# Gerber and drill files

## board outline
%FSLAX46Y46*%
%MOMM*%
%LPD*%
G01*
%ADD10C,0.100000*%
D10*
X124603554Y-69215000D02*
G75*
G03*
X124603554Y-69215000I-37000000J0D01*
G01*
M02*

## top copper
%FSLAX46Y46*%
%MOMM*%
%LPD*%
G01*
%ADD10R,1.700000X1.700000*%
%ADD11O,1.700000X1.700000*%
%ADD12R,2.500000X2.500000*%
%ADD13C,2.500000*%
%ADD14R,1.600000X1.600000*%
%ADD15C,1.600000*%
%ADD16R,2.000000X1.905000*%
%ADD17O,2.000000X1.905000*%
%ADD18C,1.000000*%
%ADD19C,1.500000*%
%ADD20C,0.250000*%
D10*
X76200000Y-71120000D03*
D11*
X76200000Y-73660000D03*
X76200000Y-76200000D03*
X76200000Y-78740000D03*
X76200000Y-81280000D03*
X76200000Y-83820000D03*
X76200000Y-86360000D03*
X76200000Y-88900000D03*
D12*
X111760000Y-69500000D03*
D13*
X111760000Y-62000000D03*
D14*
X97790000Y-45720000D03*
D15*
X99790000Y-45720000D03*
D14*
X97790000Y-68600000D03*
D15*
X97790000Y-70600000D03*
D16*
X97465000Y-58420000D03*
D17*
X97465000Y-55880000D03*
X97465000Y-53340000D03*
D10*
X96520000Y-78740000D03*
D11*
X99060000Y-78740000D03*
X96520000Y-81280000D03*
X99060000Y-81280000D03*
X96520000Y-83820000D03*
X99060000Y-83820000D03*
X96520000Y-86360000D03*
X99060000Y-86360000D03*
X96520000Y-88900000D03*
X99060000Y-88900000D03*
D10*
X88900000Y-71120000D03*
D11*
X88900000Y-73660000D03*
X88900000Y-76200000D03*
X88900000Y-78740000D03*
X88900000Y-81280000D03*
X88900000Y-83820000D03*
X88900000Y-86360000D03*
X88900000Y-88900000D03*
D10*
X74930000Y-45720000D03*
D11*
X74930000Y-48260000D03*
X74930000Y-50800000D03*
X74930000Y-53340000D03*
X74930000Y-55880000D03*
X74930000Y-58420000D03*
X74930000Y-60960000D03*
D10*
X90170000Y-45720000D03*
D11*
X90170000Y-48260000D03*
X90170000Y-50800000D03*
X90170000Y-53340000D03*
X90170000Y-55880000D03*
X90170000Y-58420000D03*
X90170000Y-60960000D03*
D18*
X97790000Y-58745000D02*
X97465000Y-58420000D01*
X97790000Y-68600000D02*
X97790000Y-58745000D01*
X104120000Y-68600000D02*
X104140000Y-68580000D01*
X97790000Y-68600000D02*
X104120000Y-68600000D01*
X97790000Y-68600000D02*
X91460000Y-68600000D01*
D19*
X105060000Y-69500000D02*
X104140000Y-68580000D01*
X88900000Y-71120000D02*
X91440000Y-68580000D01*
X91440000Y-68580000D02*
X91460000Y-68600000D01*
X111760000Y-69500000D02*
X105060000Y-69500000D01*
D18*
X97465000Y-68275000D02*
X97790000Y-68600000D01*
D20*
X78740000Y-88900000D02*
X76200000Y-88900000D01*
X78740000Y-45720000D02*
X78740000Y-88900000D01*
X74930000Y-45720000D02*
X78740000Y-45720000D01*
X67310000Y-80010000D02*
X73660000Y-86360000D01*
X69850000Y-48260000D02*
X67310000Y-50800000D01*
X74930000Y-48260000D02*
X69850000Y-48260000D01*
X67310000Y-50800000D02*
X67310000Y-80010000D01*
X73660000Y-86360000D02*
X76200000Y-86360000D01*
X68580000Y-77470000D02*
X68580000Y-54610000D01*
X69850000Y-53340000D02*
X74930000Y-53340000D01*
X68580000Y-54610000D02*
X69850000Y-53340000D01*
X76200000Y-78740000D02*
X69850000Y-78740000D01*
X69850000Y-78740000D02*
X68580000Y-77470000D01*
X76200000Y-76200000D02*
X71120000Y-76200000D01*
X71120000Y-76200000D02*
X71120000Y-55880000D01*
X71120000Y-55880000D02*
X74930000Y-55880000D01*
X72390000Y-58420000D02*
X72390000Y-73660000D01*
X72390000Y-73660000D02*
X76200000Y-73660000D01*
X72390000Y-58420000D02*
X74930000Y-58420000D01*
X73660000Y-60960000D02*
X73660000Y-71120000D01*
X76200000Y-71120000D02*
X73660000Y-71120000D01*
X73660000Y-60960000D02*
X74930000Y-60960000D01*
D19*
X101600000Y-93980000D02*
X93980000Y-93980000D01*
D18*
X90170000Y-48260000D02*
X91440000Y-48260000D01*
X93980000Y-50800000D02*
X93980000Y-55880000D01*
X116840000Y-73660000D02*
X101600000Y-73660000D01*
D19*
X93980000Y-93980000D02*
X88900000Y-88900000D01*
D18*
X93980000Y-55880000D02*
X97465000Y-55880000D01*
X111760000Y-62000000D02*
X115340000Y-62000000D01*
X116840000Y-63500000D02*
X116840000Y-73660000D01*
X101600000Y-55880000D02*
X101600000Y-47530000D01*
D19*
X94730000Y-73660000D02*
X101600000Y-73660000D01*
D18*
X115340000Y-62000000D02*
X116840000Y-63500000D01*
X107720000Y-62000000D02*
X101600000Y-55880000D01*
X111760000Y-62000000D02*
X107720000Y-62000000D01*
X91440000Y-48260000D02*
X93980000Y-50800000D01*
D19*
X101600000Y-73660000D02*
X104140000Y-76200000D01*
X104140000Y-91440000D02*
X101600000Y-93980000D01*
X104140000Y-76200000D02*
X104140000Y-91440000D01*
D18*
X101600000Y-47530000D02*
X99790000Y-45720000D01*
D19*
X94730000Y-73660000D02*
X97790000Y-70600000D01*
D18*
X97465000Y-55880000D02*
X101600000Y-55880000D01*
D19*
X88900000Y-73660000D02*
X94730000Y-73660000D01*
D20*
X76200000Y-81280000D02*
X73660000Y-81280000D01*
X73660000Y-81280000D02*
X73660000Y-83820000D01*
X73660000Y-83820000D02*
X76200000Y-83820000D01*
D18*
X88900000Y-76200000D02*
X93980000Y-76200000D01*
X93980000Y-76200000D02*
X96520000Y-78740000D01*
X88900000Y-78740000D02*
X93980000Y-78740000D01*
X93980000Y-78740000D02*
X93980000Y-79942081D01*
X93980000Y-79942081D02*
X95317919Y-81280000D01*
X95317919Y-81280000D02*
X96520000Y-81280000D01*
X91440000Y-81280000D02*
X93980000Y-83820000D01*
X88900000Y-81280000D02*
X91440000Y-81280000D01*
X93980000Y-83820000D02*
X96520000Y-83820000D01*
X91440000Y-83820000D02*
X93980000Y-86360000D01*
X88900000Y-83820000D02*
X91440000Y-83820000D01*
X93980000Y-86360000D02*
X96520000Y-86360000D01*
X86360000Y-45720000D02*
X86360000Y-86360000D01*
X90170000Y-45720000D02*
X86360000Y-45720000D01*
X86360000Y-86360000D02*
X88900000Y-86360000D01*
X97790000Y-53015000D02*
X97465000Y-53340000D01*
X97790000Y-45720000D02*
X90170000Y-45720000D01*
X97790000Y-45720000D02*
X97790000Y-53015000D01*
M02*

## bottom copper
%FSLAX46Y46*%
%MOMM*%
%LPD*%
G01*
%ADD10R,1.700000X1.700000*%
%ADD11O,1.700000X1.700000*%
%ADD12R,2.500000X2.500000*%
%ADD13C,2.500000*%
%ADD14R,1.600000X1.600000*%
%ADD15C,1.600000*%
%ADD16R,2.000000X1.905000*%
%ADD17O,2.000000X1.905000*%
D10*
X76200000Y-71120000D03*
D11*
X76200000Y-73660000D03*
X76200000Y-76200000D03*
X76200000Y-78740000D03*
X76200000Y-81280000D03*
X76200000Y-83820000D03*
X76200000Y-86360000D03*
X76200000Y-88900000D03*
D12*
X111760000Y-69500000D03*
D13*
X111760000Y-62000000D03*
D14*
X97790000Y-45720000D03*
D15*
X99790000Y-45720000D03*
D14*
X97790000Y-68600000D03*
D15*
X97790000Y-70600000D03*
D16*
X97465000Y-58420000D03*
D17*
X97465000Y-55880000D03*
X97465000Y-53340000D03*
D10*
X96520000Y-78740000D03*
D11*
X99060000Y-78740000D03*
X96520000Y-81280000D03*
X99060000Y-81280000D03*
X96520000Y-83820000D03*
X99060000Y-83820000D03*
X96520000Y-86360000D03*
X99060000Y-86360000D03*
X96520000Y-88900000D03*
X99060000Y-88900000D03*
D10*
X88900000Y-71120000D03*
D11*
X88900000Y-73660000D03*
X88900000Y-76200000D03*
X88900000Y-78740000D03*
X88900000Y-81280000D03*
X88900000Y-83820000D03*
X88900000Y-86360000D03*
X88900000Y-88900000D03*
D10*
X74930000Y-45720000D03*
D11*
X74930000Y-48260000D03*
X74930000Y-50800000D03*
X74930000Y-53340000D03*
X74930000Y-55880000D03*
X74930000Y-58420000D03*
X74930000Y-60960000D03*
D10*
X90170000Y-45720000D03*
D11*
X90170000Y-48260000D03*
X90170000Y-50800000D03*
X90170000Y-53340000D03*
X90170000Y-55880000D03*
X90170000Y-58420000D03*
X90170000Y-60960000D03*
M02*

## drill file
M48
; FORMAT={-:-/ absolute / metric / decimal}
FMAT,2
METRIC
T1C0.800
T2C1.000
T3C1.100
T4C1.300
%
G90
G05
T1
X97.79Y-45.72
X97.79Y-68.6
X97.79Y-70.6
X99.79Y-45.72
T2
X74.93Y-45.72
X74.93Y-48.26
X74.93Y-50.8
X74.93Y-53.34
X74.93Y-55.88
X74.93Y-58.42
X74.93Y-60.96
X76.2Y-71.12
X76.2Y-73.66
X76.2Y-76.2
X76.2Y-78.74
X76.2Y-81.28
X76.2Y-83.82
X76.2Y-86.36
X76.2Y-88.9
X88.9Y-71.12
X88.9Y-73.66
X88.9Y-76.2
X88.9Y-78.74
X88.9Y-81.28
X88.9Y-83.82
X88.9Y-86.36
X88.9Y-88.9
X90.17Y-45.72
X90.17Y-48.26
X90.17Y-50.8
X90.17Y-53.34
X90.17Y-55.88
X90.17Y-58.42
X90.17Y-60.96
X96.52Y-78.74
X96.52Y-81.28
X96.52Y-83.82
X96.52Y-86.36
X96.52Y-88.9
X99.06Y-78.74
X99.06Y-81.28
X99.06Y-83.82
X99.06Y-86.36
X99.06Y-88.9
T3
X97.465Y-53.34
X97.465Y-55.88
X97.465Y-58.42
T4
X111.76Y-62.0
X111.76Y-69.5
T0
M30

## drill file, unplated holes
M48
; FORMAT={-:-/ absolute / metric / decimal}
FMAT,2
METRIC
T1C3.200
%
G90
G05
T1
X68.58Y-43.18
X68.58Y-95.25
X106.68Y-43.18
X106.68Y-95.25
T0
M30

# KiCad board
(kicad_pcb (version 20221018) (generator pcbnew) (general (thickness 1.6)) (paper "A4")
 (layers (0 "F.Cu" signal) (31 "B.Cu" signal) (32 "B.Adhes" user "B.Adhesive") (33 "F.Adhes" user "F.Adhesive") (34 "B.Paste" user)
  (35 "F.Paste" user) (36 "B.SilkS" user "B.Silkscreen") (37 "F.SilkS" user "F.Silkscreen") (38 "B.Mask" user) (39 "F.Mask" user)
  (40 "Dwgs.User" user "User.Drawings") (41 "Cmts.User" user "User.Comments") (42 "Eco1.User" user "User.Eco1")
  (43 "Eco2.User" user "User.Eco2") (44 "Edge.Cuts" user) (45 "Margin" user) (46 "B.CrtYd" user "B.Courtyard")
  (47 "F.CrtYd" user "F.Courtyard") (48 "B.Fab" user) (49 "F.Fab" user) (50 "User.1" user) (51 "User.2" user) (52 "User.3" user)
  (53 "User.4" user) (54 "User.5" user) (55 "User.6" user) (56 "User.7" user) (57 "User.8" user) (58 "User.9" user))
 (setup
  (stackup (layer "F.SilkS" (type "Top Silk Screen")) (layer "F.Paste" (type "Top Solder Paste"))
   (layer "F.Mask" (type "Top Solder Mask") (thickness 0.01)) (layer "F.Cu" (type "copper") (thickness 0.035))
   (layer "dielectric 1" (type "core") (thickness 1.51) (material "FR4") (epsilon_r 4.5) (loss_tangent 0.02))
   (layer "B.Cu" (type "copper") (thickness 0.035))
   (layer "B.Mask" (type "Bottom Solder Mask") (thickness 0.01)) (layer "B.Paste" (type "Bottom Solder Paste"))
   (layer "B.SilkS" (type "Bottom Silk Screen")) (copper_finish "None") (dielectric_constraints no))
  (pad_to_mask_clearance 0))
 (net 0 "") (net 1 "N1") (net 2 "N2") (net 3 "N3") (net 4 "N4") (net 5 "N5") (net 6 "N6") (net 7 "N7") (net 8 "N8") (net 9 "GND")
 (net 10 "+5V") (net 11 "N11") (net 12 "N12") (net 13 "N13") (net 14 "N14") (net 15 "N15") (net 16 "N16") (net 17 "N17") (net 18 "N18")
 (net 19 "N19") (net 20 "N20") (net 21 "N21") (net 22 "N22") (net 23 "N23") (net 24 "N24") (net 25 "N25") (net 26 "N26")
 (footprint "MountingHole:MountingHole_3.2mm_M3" (layer "F.Cu") (at 106.68 95.25)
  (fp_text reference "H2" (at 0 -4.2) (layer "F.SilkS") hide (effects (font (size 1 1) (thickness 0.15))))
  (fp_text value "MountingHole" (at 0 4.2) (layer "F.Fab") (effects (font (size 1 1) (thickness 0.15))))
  (pad "" np_thru_hole circle (at 0 0) (size 3.2 3.2) (drill 3.2) (layers "*.Cu" "*.Mask")))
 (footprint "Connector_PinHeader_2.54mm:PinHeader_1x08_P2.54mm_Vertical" (layer "F.Cu") (at 76.2 71.12)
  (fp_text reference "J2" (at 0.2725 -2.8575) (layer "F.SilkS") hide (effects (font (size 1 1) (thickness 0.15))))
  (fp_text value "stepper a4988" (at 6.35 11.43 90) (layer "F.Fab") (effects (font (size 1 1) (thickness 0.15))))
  (pad "1" thru_hole rect (at 0 0) (size 1.7 1.7) (drill 1) (layers "*.Cu" "*.Mask") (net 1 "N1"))
  (pad "2" thru_hole oval (at 0 2.54) (size 1.7 1.7) (drill 1) (layers "*.Cu" "*.Mask") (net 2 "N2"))
  (pad "3" thru_hole oval (at 0 5.08) (size 1.7 1.7) (drill 1) (layers "*.Cu" "*.Mask") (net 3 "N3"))
  (pad "4" thru_hole oval (at 0 7.62) (size 1.7 1.7) (drill 1) (layers "*.Cu" "*.Mask") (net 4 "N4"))
  (pad "5" thru_hole oval (at 0 10.16) (size 1.7 1.7) (drill 1) (layers "*.Cu" "*.Mask") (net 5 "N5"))
  (pad "6" thru_hole oval (at 0 12.7) (size 1.7 1.7) (drill 1) (layers "*.Cu" "*.Mask") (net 5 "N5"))
  (pad "7" thru_hole oval (at 0 15.24) (size 1.7 1.7) (drill 1) (layers "*.Cu" "*.Mask") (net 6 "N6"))
  (pad "8" thru_hole oval (at 0 17.78) (size 1.7 1.7) (drill 1) (layers "*.Cu" "*.Mask") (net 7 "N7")))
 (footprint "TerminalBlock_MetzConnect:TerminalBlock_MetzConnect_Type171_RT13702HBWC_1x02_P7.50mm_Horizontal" (layer "F.Cu")
  (at 111.76 69.5 90)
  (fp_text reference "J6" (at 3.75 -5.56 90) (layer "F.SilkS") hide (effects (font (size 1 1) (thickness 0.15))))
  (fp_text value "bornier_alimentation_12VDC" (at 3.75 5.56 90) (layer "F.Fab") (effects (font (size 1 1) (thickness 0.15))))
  (pad "1" thru_hole rect (at 0 0 90) (size 2.5 2.5) (drill 1.3) (layers "*.Cu" "*.Mask") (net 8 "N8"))
  (pad "2" thru_hole circle (at 7.5 0 90) (size 2.5 2.5) (drill 1.3) (layers "*.Cu" "*.Mask") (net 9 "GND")))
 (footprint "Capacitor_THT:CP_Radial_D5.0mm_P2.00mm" (layer "F.Cu") (at 97.79 45.72)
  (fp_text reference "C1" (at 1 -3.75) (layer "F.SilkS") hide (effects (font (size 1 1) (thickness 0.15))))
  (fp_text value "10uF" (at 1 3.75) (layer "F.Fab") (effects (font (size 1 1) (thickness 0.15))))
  (pad "1" thru_hole rect (at 0 0) (size 1.6 1.6) (drill 0.8) (layers "*.Cu" "*.Mask") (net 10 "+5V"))
  (pad "2" thru_hole circle (at 2 0) (size 1.6 1.6) (drill 0.8) (layers "*.Cu" "*.Mask") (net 9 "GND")))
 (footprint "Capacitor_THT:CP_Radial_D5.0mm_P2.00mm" (layer "F.Cu") (at 97.79 68.6 -90)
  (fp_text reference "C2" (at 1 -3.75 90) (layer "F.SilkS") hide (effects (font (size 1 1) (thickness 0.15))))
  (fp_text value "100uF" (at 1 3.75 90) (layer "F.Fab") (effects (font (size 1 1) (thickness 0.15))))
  (pad "1" thru_hole rect (at 0 0 270) (size 1.6 1.6) (drill 0.8) (layers "*.Cu" "*.Mask") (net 8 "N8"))
  (pad "2" thru_hole circle (at 2 0 270) (size 1.6 1.6) (drill 0.8) (layers "*.Cu" "*.Mask") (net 9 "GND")))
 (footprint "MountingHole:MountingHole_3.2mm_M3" (layer "F.Cu") (at 68.58 43.18)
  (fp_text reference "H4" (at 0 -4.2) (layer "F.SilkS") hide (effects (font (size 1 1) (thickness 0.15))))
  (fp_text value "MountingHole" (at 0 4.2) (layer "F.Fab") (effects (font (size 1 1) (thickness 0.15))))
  (pad "" np_thru_hole circle (at 0 0) (size 3.2 3.2) (drill 3.2) (layers "*.Cu" "*.Mask")))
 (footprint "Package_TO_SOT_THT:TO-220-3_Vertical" (layer "F.Cu") (at 97.465 58.42 90)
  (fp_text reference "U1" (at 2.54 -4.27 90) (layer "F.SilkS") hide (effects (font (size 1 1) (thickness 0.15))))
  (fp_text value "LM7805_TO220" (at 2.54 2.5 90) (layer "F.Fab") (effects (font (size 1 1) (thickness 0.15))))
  (pad "1" thru_hole rect (at 0 0 90) (size 1.905 2) (drill 1.1) (layers "*.Cu" "*.Mask") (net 8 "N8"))
  (pad "2" thru_hole oval (at 2.54 0 90) (size 1.905 2) (drill 1.1) (layers "*.Cu" "*.Mask") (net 9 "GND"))
  (pad "3" thru_hole oval (at 5.08 0 90) (size 1.905 2) (drill 1.1) (layers "*.Cu" "*.Mask") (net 10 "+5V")))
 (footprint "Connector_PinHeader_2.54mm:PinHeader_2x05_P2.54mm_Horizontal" (layer "F.Cu") (at 96.52 78.74)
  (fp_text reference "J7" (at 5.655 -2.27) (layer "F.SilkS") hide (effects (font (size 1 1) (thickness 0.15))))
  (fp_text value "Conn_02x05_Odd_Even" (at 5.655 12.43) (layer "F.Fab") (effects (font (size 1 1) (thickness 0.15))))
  (pad "1" thru_hole rect (at 0 0) (size 1.7 1.7) (drill 1) (layers "*.Cu" "*.Mask") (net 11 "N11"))
  (pad "2" thru_hole oval (at 2.54 0) (size 1.7 1.7) (drill 1) (layers "*.Cu" "*.Mask") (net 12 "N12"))
  (pad "3" thru_hole oval (at 0 2.54) (size 1.7 1.7) (drill 1) (layers "*.Cu" "*.Mask") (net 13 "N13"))
  (pad "4" thru_hole oval (at 2.54 2.54) (size 1.7 1.7) (drill 1) (layers "*.Cu" "*.Mask") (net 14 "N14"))
  (pad "5" thru_hole oval (at 0 5.08) (size 1.7 1.7) (drill 1) (layers "*.Cu" "*.Mask") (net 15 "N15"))
  (pad "6" thru_hole oval (at 2.54 5.08) (size 1.7 1.7) (drill 1) (layers "*.Cu" "*.Mask") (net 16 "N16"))
  (pad "7" thru_hole oval (at 0 7.62) (size 1.7 1.7) (drill 1) (layers "*.Cu" "*.Mask") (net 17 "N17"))
  (pad "8" thru_hole oval (at 2.54 7.62) (size 1.7 1.7) (drill 1) (layers "*.Cu" "*.Mask") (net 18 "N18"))
  (pad "9" thru_hole oval (at 0 10.16) (size 1.7 1.7) (drill 1) (layers "*.Cu" "*.Mask") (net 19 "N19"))
  (pad "10" thru_hole oval (at 2.54 10.16) (size 1.7 1.7) (drill 1) (layers "*.Cu" "*.Mask") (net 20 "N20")))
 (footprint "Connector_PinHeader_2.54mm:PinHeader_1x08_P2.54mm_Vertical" (layer "F.Cu") (at 88.9 71.12)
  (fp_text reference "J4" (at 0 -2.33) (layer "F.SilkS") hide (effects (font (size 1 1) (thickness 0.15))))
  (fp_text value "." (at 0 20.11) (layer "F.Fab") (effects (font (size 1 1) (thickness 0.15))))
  (pad "1" thru_hole rect (at 0 0) (size 1.7 1.7) (drill 1) (layers "*.Cu" "*.Mask") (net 8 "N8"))
  (pad "2" thru_hole oval (at 0 2.54) (size 1.7 1.7) (drill 1) (layers "*.Cu" "*.Mask") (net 9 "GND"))
  (pad "3" thru_hole oval (at 0 5.08) (size 1.7 1.7) (drill 1) (layers "*.Cu" "*.Mask") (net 11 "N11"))
  (pad "4" thru_hole oval (at 0 7.62) (size 1.7 1.7) (drill 1) (layers "*.Cu" "*.Mask") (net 13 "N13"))
  (pad "5" thru_hole oval (at 0 10.16) (size 1.7 1.7) (drill 1) (layers "*.Cu" "*.Mask") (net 15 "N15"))
  (pad "6" thru_hole oval (at 0 12.7) (size 1.7 1.7) (drill 1) (layers "*.Cu" "*.Mask") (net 17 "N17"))
  (pad "7" thru_hole oval (at 0 15.24) (size 1.7 1.7) (drill 1) (layers "*.Cu" "*.Mask") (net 10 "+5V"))
  (pad "8" thru_hole oval (at 0 17.78) (size 1.7 1.7) (drill 1) (layers "*.Cu" "*.Mask") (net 9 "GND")))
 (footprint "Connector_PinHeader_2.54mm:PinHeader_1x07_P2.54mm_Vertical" (layer "F.Cu") (at 74.93 45.72)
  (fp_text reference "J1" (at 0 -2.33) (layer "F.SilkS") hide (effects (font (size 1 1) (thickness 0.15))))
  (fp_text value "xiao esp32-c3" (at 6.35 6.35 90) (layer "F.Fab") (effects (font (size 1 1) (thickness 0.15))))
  (pad "1" thru_hole rect (at 0 0) (size 1.7 1.7) (drill 1) (layers "*.Cu" "*.Mask") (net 7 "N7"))
  (pad "2" thru_hole oval (at 0 2.54) (size 1.7 1.7) (drill 1) (layers "*.Cu" "*.Mask") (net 6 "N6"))
  (pad "3" thru_hole oval (at 0 5.08) (size 1.7 1.7) (drill 1) (layers "*.Cu" "*.Mask") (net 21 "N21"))
  (pad "4" thru_hole oval (at 0 7.62) (size 1.7 1.7) (drill 1) (layers "*.Cu" "*.Mask") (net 4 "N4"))
  (pad "5" thru_hole oval (at 0 10.16) (size 1.7 1.7) (drill 1) (layers "*.Cu" "*.Mask") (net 3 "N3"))
  (pad "6" thru_hole oval (at 0 12.7) (size 1.7 1.7) (drill 1) (layers "*.Cu" "*.Mask") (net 2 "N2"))
  (pad "7" thru_hole oval (at 0 15.24) (size 1.7 1.7) (drill 1) (layers "*.Cu" "*.Mask") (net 1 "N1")))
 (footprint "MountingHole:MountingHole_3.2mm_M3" (layer "F.Cu") (at 106.68 43.18)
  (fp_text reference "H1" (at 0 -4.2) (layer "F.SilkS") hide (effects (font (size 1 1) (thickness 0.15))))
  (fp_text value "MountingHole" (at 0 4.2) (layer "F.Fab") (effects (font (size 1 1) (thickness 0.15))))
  (pad "" np_thru_hole circle (at 0 0) (size 3.2 3.2) (drill 3.2) (layers "*.Cu" "*.Mask")))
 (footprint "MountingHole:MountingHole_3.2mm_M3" (layer "F.Cu") (at 68.58 95.25)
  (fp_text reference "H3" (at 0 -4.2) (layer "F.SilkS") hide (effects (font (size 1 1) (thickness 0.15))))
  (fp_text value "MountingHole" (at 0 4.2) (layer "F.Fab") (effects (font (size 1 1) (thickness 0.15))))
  (pad "" np_thru_hole circle (at 0 0) (size 3.2 3.2) (drill 3.2) (layers "*.Cu" "*.Mask")))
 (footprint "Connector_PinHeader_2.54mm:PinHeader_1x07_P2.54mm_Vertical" (layer "F.Cu") (at 90.17 45.72)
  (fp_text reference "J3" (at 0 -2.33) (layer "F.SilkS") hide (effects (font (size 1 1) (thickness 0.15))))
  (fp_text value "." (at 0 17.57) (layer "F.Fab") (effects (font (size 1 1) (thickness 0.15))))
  (pad "1" thru_hole rect (at 0 0) (size 1.7 1.7) (drill 1) (layers "*.Cu" "*.Mask") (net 10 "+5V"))
  (pad "2" thru_hole oval (at 0 2.54) (size 1.7 1.7) (drill 1) (layers "*.Cu" "*.Mask") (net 9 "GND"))
  (pad "3" thru_hole oval (at 0 5.08) (size 1.7 1.7) (drill 1) (layers "*.Cu" "*.Mask") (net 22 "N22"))
  (pad "4" thru_hole oval (at 0 7.62) (size 1.7 1.7) (drill 1) (layers "*.Cu" "*.Mask") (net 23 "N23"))
  (pad "5" thru_hole oval (at 0 10.16) (size 1.7 1.7) (drill 1) (layers "*.Cu" "*.Mask") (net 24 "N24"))
  (pad "6" thru_hole oval (at 0 12.7) (size 1.7 1.7) (drill 1) (layers "*.Cu" "*.Mask") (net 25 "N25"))
  (pad "7" thru_hole oval (at 0 15.24) (size 1.7 1.7) (drill 1) (layers "*.Cu" "*.Mask") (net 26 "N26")))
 (gr_circle (center 87.603554 69.215) (end 124.603554 69.215) (stroke (width 0.1) (type solid)) (fill none) (layer "Edge.Cuts"))
 (segment (start 105.06 69.5) (end 104.14 68.58) (width 1.5) (layer "F.Cu") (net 8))
 (segment (start 97.79 68.6) (end 104.12 68.6) (width 1) (layer "F.Cu") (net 8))
 (segment (start 88.9 71.12) (end 91.44 68.58) (width 1.5) (layer "F.Cu") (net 8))
 (segment (start 104.12 68.6) (end 104.14 68.58) (width 1) (layer "F.Cu") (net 8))
 (segment (start 91.44 68.58) (end 91.46 68.6) (width 1.5) (layer "F.Cu") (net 8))
 (segment (start 111.76 69.5) (end 105.06 69.5) (width 1.5) (layer "F.Cu") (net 8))
 (segment (start 97.465 68.275) (end 97.79 68.6) (width 1) (layer "F.Cu") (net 8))
 (segment (start 97.79 68.6) (end 91.46 68.6) (width 1) (layer "F.Cu") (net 8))
 (segment (start 97.79 68.6) (end 97.79 58.745) (width 1) (layer "F.Cu") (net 8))
 (segment (start 97.79 58.745) (end 97.465 58.42) (width 1) (layer "F.Cu") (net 8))
 (segment (start 78.74 88.9) (end 76.2 88.9) (width 0.25) (layer "F.Cu") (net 7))
 (segment (start 78.74 45.72) (end 78.74 88.9) (width 0.25) (layer "F.Cu") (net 7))
 (segment (start 74.93 45.72) (end 78.74 45.72) (width 0.25) (layer "F.Cu") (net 7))
 (segment (start 67.31 80.01) (end 73.66 86.36) (width 0.25) (layer "F.Cu") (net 6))
 (segment (start 69.85 48.26) (end 67.31 50.8) (width 0.25) (layer "F.Cu") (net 6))
 (segment (start 74.93 48.26) (end 69.85 48.26) (width 0.25) (layer "F.Cu") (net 6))
 (segment (start 67.31 50.8) (end 67.31 80.01) (width 0.25) (layer "F.Cu") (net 6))
 (segment (start 73.66 86.36) (end 76.2 86.36) (width 0.25) (layer "F.Cu") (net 6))
 (segment (start 68.58 77.47) (end 68.58 54.61) (width 0.25) (layer "F.Cu") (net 4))
 (segment (start 69.85 53.34) (end 74.93 53.34) (width 0.25) (layer "F.Cu") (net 4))
 (segment (start 68.58 54.61) (end 69.85 53.34) (width 0.25) (layer "F.Cu") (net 4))
 (segment (start 76.2 78.74) (end 69.85 78.74) (width 0.25) (layer "F.Cu") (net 4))
 (segment (start 69.85 78.74) (end 68.58 77.47) (width 0.25) (layer "F.Cu") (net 4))
 (segment (start 76.2 76.2) (end 71.12 76.2) (width 0.25) (layer "F.Cu") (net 3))
 (segment (start 71.12 76.2) (end 71.12 55.88) (width 0.25) (layer "F.Cu") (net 3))
 (segment (start 71.12 55.88) (end 74.93 55.88) (width 0.25) (layer "F.Cu") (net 3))
 (segment (start 72.39 58.42) (end 72.39 73.66) (width 0.25) (layer "F.Cu") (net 2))
 (segment (start 72.39 73.66) (end 76.2 73.66) (width 0.25) (layer "F.Cu") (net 2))
 (segment (start 72.39 58.42) (end 74.93 58.42) (width 0.25) (layer "F.Cu") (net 2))
 (segment (start 73.66 60.96) (end 73.66 71.12) (width 0.25) (layer "F.Cu") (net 1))
 (segment (start 76.2 71.12) (end 73.66 71.12) (width 0.25) (layer "F.Cu") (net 1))
 (segment (start 73.66 60.96) (end 74.93 60.96) (width 0.25) (layer "F.Cu") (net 1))
 (segment (start 101.6 93.98) (end 93.98 93.98) (width 1.5) (layer "F.Cu") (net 9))
 (segment (start 90.17 48.26) (end 91.44 48.26) (width 1) (layer "F.Cu") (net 9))
 (segment (start 93.98 50.8) (end 93.98 55.88) (width 1) (layer "F.Cu") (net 9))
 (segment (start 116.84 73.66) (end 101.6 73.66) (width 1) (layer "F.Cu") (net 9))
 (segment (start 93.98 93.98) (end 88.9 88.9) (width 1.5) (layer "F.Cu") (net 9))
 (segment (start 93.98 55.88) (end 97.465 55.88) (width 1) (layer "F.Cu") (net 9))
 (segment (start 111.76 62) (end 115.34 62) (width 1) (layer "F.Cu") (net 9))
 (segment (start 116.84 63.5) (end 116.84 73.66) (width 1) (layer "F.Cu") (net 9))
 (segment (start 101.6 55.88) (end 101.6 47.53) (width 1) (layer "F.Cu") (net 9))
 (segment (start 94.73 73.66) (end 101.6 73.66) (width 1.5) (layer "F.Cu") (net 9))
 (segment (start 115.34 62) (end 116.84 63.5) (width 1) (layer "F.Cu") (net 9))
 (segment (start 107.72 62) (end 101.6 55.88) (width 1) (layer "F.Cu") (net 9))
 (segment (start 111.76 62) (end 107.72 62) (width 1) (layer "F.Cu") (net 9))
 (segment (start 91.44 48.26) (end 93.98 50.8) (width 1) (layer "F.Cu") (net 9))
 (segment (start 101.6 73.66) (end 104.14 76.2) (width 1.5) (layer "F.Cu") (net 9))
 (segment (start 104.14 91.44) (end 101.6 93.98) (width 1.5) (layer "F.Cu") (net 9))
 (segment (start 104.14 76.2) (end 104.14 91.44) (width 1.5) (layer "F.Cu") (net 9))
 (segment (start 101.6 47.53) (end 99.79 45.72) (width 1) (layer "F.Cu") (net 9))
 (segment (start 94.73 73.66) (end 97.79 70.6) (width 1.5) (layer "F.Cu") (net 9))
 (segment (start 97.465 55.88) (end 101.6 55.88) (width 1) (layer "F.Cu") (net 9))
 (segment (start 88.9 73.66) (end 94.73 73.66) (width 1.5) (layer "F.Cu") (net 9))
 (segment (start 76.2 81.28) (end 73.66 81.28) (width 0.25) (layer "F.Cu") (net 5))
 (segment (start 73.66 81.28) (end 73.66 83.82) (width 0.25) (layer "F.Cu") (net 5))
 (segment (start 73.66 83.82) (end 76.2 83.82) (width 0.25) (layer "F.Cu") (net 5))
 (segment (start 88.9 76.2) (end 93.98 76.2) (width 1) (layer "F.Cu") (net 11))
 (segment (start 93.98 76.2) (end 96.52 78.74) (width 1) (layer "F.Cu") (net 11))
 (segment (start 88.9 78.74) (end 93.98 78.74) (width 1) (layer "F.Cu") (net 13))
 (segment (start 93.98 78.74) (end 93.98 79.942081) (width 1) (layer "F.Cu") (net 13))
 (segment (start 93.98 79.942081) (end 95.317919 81.28) (width 1) (layer "F.Cu") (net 13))
 (segment (start 95.317919 81.28) (end 96.52 81.28) (width 1) (layer "F.Cu") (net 13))
 (segment (start 91.44 81.28) (end 93.98 83.82) (width 1) (layer "F.Cu") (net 15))
 (segment (start 88.9 81.28) (end 91.44 81.28) (width 1) (layer "F.Cu") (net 15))
 (segment (start 93.98 83.82) (end 96.52 83.82) (width 1) (layer "F.Cu") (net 15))
 (segment (start 91.44 83.82) (end 93.98 86.36) (width 1) (layer "F.Cu") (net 17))
 (segment (start 88.9 83.82) (end 91.44 83.82) (width 1) (layer "F.Cu") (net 17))
 (segment (start 93.98 86.36) (end 96.52 86.36) (width 1) (layer "F.Cu") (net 17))
 (segment (start 86.36 45.72) (end 86.36 86.36) (width 1) (layer "F.Cu") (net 10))
 (segment (start 90.17 45.72) (end 86.36 45.72) (width 1) (layer "F.Cu") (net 10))
 (segment (start 86.36 86.36) (end 88.9 86.36) (width 1) (layer "F.Cu") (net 10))
 (segment (start 97.79 53.015) (end 97.465 53.34) (width 1) (layer "F.Cu") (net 10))
 (segment (start 97.79 45.72) (end 90.17 45.72) (width 1) (layer "F.Cu") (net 10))
 (segment (start 97.79 45.72) (end 97.79 53.015) (width 1) (layer "F.Cu") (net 10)))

